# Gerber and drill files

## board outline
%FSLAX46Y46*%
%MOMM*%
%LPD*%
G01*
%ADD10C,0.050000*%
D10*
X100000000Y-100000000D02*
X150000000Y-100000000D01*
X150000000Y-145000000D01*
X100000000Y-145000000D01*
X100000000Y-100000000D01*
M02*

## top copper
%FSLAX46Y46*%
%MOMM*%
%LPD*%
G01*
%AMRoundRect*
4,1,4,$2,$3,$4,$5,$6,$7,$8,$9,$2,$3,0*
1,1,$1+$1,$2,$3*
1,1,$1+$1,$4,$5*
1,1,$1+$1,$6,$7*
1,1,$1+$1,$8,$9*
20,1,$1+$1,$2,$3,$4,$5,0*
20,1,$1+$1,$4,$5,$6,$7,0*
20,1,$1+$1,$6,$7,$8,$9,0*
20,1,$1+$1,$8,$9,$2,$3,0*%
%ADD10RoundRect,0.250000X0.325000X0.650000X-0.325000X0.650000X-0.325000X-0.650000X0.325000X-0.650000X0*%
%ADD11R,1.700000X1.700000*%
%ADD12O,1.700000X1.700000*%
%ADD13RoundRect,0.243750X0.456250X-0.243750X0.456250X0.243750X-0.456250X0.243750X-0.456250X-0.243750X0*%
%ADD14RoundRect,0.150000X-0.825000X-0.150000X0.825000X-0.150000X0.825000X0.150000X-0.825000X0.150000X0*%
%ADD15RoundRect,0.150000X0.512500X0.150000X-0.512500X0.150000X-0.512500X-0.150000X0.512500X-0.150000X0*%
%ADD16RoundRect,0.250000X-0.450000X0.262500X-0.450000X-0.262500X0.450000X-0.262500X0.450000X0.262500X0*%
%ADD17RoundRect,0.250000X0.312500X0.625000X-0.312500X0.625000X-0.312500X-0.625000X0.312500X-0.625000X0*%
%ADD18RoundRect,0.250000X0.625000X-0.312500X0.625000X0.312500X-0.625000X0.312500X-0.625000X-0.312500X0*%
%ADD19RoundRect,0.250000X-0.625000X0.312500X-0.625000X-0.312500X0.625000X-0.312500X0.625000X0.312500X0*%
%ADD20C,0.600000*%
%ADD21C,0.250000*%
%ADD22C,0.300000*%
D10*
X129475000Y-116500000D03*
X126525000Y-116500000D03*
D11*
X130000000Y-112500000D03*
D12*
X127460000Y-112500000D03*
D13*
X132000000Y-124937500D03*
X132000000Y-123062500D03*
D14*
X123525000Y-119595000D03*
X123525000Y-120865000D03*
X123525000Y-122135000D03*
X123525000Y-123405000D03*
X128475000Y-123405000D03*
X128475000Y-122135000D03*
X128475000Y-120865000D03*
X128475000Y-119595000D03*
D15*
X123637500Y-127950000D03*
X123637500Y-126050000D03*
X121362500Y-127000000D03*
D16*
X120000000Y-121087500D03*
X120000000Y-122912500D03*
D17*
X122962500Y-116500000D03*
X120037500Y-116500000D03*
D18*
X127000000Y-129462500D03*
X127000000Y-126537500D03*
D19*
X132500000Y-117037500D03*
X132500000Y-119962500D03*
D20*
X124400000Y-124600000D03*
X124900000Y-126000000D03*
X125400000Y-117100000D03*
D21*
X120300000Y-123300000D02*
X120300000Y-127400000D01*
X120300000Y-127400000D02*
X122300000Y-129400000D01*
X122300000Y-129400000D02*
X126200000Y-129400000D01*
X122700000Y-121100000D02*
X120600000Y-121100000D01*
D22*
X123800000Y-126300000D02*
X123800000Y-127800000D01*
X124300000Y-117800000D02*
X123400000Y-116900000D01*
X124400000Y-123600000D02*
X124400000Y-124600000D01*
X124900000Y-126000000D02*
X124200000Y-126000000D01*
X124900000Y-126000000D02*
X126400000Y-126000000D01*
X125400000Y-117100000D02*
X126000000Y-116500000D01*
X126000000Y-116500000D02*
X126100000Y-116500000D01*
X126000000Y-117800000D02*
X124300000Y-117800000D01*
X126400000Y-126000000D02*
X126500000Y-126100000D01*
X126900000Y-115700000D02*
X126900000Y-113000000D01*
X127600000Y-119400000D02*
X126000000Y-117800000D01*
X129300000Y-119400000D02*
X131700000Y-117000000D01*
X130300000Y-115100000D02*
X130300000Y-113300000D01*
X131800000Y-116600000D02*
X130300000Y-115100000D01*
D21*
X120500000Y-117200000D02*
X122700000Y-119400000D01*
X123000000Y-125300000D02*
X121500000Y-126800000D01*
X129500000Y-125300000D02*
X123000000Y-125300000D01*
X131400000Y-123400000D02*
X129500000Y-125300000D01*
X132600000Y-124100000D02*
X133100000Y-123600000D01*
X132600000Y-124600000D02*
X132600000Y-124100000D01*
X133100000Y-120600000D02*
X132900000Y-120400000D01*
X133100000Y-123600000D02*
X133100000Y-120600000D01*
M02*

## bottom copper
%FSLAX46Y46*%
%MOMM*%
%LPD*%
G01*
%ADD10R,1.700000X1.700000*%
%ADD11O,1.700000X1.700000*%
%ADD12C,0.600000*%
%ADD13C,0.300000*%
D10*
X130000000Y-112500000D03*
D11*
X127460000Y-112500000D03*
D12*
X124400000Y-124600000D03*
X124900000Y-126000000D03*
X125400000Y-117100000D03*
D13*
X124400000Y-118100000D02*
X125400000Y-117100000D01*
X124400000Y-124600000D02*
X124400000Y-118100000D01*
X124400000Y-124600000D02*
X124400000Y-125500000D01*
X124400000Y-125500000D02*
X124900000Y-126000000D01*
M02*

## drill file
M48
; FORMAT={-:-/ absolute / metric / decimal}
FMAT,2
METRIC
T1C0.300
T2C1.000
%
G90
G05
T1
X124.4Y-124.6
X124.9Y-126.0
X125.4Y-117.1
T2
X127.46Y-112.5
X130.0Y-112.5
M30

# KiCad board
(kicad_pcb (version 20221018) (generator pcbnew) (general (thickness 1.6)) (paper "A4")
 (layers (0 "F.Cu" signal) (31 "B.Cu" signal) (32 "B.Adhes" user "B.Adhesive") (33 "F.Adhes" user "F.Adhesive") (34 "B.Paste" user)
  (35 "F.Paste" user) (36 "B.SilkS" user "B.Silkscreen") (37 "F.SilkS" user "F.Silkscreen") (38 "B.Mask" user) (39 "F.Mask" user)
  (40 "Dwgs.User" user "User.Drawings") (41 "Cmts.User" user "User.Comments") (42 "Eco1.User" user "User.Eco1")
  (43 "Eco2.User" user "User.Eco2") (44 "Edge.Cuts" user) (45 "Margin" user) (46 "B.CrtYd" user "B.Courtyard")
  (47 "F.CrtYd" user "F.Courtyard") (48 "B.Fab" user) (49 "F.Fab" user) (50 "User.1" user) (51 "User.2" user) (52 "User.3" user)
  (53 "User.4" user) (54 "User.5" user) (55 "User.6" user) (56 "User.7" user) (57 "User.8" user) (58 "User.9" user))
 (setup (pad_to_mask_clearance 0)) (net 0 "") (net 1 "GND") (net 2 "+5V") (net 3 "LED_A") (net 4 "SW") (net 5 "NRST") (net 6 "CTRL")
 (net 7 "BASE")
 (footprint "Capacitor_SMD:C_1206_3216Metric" (layer "F.Cu") (at 128 116.5 180)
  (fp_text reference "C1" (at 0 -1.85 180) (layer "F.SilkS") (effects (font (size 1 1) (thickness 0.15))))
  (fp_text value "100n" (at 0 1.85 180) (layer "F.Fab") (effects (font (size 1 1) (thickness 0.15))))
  (pad "1" smd roundrect (at -1.475 0 180) (size 1.15 1.8) (layers "F.Cu" "F.Paste" "F.Mask") (roundrect_rratio 0.217391))
  (pad "2" smd roundrect (at 1.475 0 180) (size 1.15 1.8) (layers "F.Cu" "F.Paste" "F.Mask") (roundrect_rratio 0.217391) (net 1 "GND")))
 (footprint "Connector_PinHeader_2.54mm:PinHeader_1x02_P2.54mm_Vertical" (layer "F.Cu") (at 130 112.5 -90)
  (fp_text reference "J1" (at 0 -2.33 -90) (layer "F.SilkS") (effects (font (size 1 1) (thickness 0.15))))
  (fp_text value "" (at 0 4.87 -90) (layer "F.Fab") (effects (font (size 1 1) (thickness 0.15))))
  (pad "1" thru_hole rect (at 0 0 270) (size 1.7 1.7) (drill 1) (layers "*.Cu" "*.Mask") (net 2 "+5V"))
  (pad "2" thru_hole oval (at 0 2.54 270) (size 1.7 1.7) (drill 1) (layers "*.Cu" "*.Mask") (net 1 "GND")))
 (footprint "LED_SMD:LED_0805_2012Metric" (layer "F.Cu") (at 132 124 90)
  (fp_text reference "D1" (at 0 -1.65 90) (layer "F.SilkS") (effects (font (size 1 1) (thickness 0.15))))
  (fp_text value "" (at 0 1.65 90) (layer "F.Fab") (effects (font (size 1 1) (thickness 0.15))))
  (pad "1" smd roundrect (at -0.9375 0 90) (size 0.975 1.4) (layers "F.Cu" "F.Paste" "F.Mask") (roundrect_rratio 0.25) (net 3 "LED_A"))
  (pad "2" smd roundrect (at 0.9375 0 90) (size 0.975 1.4) (layers "F.Cu" "F.Paste" "F.Mask") (roundrect_rratio 0.25) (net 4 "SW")))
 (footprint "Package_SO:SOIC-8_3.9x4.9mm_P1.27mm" (layer "F.Cu") (at 126 121.5)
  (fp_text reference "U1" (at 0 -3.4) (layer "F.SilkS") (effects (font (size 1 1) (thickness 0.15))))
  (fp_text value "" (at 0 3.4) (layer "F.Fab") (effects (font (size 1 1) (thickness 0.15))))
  (pad "1" smd roundrect (at -2.475 -1.905) (size 1.95 0.6) (layers "F.Cu" "F.Paste" "F.Mask") (roundrect_rratio 0.25) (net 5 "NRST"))
  (pad "2" smd roundrect (at -2.475 -0.635) (size 1.95 0.6) (layers "F.Cu" "F.Paste" "F.Mask") (roundrect_rratio 0.25) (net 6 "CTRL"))
  (pad "3" smd roundrect (at -2.475 0.635) (size 1.95 0.6) (layers "F.Cu" "F.Paste" "F.Mask") (roundrect_rratio 0.25))
  (pad "4" smd roundrect (at -2.475 1.905) (size 1.95 0.6) (layers "F.Cu" "F.Paste" "F.Mask") (roundrect_rratio 0.25) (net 1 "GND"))
  (pad "5" smd roundrect (at 2.475 1.905) (size 1.95 0.6) (layers "F.Cu" "F.Paste" "F.Mask") (roundrect_rratio 0.25))
  (pad "6" smd roundrect (at 2.475 0.635) (size 1.95 0.6) (layers "F.Cu" "F.Paste" "F.Mask") (roundrect_rratio 0.25))
  (pad "7" smd roundrect (at 2.475 -0.635) (size 1.95 0.6) (layers "F.Cu" "F.Paste" "F.Mask") (roundrect_rratio 0.25))
  (pad "8" smd roundrect (at 2.475 -1.905) (size 1.95 0.6) (layers "F.Cu" "F.Paste" "F.Mask") (roundrect_rratio 0.25) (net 2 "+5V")))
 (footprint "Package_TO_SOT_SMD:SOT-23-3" (layer "F.Cu") (at 122.5 127 180)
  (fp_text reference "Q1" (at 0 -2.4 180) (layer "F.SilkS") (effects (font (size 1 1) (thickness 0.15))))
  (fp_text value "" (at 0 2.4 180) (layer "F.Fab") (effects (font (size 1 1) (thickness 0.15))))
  (pad "1" smd roundrect (at -1.1375 -0.95 180) (size 1.325 0.6) (layers "F.Cu" "F.Paste" "F.Mask") (roundrect_rratio 0.25) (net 1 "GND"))
  (pad "2" smd roundrect (at -1.1375 0.95 180) (size 1.325 0.6) (layers "F.Cu" "F.Paste" "F.Mask") (roundrect_rratio 0.25) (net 1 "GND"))
  (pad "3" smd roundrect (at 1.1375 0 180) (size 1.325 0.6) (layers "F.Cu" "F.Paste" "F.Mask") (roundrect_rratio 0.25) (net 4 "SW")))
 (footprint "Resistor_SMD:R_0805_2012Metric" (layer "F.Cu") (at 120 122 -90)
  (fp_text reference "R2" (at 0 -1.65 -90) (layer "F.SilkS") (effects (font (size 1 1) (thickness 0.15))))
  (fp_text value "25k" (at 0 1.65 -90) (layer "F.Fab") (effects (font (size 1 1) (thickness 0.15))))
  (pad "1" smd roundrect (at -0.9125 0 270) (size 1.025 1.4) (layers "F.Cu" "F.Paste" "F.Mask") (roundrect_rratio 0.243902) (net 6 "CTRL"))
  (pad "2" smd roundrect (at 0.9125 0 270) (size 1.025 1.4) (layers "F.Cu" "F.Paste" "F.Mask") (roundrect_rratio 0.243902) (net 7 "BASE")))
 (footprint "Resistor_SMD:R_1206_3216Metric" (layer "F.Cu") (at 121.5 116.5 180)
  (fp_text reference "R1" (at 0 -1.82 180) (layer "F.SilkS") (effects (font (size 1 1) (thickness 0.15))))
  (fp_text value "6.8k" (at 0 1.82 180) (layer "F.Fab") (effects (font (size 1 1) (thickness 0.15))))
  (pad "1" smd roundrect (at -1.4625 0 180) (size 1.125 1.75) (layers "F.Cu" "F.Paste" "F.Mask") (roundrect_rratio 0.222222) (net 2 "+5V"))
  (pad "2" smd roundrect (at 1.4625 0 180) (size 1.125 1.75) (layers "F.Cu" "F.Paste" "F.Mask") (roundrect_rratio 0.222222) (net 5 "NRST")))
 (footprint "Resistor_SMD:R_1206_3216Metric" (layer "F.Cu") (at 127 128 90)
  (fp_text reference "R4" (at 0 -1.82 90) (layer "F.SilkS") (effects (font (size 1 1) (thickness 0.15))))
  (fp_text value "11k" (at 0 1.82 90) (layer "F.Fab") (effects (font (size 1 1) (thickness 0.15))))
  (pad "1" smd roundrect (at -1.4625 0 90) (size 1.125 1.75) (layers "F.Cu" "F.Paste" "F.Mask") (roundrect_rratio 0.222222) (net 7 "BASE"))
  (pad "2" smd roundrect (at 1.4625 0 90) (size 1.125 1.75) (layers "F.Cu" "F.Paste" "F.Mask") (roundrect_rratio 0.222222) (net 1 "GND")))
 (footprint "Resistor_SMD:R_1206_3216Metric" (layer "F.Cu") (at 132.5 118.5 -90)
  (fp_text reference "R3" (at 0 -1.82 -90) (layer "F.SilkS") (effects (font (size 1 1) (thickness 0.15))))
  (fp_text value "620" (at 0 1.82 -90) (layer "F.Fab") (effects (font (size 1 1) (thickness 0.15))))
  (pad "1" smd roundrect (at -1.4625 0 270) (size 1.125 1.75) (layers "F.Cu" "F.Paste" "F.Mask") (roundrect_rratio 0.222222) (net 2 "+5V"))
  (pad "2" smd roundrect (at 1.4625 0 270) (size 1.125 1.75) (layers "F.Cu" "F.Paste" "F.Mask") (roundrect_rratio 0.222222) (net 3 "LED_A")))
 (gr_rect (start 100 100) (end 150 145) (stroke (width 0.05) (type default)) (fill none) (layer "Edge.Cuts"))
 (segment (start 120.3 123.3) (end 120.3 127.4) (width 0.25) (layer "F.Cu") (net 7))
 (segment (start 120.3 127.4) (end 122.3 129.4) (width 0.25) (layer "F.Cu") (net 7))
 (segment (start 122.3 129.4) (end 126.2 129.4) (width 0.25) (layer "F.Cu") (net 7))
 (segment (start 122.7 121.1) (end 120.6 121.1) (width 0.25) (layer "F.Cu") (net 6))
 (segment (start 123.8 126.3) (end 123.8 127.8) (width 0.3) (layer "F.Cu") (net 1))
 (segment (start 124.3 117.8) (end 123.4 116.9) (width 0.3) (layer "F.Cu") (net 2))
 (segment (start 124.4 123.6) (end 124.4 124.6) (width 0.3) (layer "F.Cu") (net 1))
 (segment (start 124.9 126) (end 124.2 126) (width 0.3) (layer "F.Cu") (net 1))
 (segment (start 124.9 126) (end 126.4 126) (width 0.3) (layer "F.Cu") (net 1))
 (segment (start 125.4 117.1) (end 126 116.5) (width 0.3) (layer "F.Cu") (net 1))
 (segment (start 126 116.5) (end 126.1 116.5) (width 0.3) (layer "F.Cu") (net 1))
 (segment (start 126 117.8) (end 124.3 117.8) (width 0.3) (layer "F.Cu") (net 2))
 (segment (start 126.4 126) (end 126.5 126.1) (width 0.3) (layer "F.Cu") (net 1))
 (segment (start 126.9 115.7) (end 126.9 113) (width 0.3) (layer "F.Cu") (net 1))
 (segment (start 127.6 119.4) (end 126 117.8) (width 0.3) (layer "F.Cu") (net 2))
 (segment (start 129.3 119.4) (end 131.7 117) (width 0.3) (layer "F.Cu") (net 2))
 (segment (start 130.3 115.1) (end 130.3 113.3) (width 0.3) (layer "F.Cu") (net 2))
 (segment (start 131.8 116.6) (end 130.3 115.1) (width 0.3) (layer "F.Cu") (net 2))
 (via (at 124.4 124.6) (size 0.6) (drill 0.3) (layers "F.Cu" "B.Cu") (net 1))
 (via (at 124.9 126) (size 0.6) (drill 0.3) (layers "F.Cu" "B.Cu") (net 1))
 (via (at 125.4 117.1) (size 0.6) (drill 0.3) (layers "F.Cu" "B.Cu") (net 1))
 (segment (start 120.5 117.2) (end 122.7 119.4) (width 0.25) (layer "F.Cu") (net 5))
 (segment (start 123 125.3) (end 121.5 126.8) (width 0.25) (layer "F.Cu") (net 4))
 (segment (start 124.4 118.1) (end 125.4 117.1) (width 0.3) (layer "B.Cu") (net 1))
 (segment (start 124.4 124.6) (end 124.4 118.1) (width 0.3) (layer "B.Cu") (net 1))
 (segment (start 124.4 124.6) (end 124.4 125.5) (width 0.3) (layer "B.Cu") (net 1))
 (segment (start 124.4 125.5) (end 124.9 126) (width 0.3) (layer "B.Cu") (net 1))
 (segment (start 129.5 125.3) (end 123 125.3) (width 0.25) (layer "F.Cu") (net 4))
 (segment (start 131.4 123.4) (end 129.5 125.3) (width 0.25) (layer "F.Cu") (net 4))
 (segment (start 132.6 124.1) (end 133.1 123.6) (width 0.25) (layer "F.Cu") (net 3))
 (segment (start 132.6 124.6) (end 132.6 124.1) (width 0.25) (layer "F.Cu") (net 3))
 (segment (start 133.1 120.6) (end 132.9 120.4) (width 0.25) (layer "F.Cu") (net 3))
 (segment (start 133.1 123.6) (end 133.1 120.6) (width 0.25) (layer "F.Cu") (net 3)))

